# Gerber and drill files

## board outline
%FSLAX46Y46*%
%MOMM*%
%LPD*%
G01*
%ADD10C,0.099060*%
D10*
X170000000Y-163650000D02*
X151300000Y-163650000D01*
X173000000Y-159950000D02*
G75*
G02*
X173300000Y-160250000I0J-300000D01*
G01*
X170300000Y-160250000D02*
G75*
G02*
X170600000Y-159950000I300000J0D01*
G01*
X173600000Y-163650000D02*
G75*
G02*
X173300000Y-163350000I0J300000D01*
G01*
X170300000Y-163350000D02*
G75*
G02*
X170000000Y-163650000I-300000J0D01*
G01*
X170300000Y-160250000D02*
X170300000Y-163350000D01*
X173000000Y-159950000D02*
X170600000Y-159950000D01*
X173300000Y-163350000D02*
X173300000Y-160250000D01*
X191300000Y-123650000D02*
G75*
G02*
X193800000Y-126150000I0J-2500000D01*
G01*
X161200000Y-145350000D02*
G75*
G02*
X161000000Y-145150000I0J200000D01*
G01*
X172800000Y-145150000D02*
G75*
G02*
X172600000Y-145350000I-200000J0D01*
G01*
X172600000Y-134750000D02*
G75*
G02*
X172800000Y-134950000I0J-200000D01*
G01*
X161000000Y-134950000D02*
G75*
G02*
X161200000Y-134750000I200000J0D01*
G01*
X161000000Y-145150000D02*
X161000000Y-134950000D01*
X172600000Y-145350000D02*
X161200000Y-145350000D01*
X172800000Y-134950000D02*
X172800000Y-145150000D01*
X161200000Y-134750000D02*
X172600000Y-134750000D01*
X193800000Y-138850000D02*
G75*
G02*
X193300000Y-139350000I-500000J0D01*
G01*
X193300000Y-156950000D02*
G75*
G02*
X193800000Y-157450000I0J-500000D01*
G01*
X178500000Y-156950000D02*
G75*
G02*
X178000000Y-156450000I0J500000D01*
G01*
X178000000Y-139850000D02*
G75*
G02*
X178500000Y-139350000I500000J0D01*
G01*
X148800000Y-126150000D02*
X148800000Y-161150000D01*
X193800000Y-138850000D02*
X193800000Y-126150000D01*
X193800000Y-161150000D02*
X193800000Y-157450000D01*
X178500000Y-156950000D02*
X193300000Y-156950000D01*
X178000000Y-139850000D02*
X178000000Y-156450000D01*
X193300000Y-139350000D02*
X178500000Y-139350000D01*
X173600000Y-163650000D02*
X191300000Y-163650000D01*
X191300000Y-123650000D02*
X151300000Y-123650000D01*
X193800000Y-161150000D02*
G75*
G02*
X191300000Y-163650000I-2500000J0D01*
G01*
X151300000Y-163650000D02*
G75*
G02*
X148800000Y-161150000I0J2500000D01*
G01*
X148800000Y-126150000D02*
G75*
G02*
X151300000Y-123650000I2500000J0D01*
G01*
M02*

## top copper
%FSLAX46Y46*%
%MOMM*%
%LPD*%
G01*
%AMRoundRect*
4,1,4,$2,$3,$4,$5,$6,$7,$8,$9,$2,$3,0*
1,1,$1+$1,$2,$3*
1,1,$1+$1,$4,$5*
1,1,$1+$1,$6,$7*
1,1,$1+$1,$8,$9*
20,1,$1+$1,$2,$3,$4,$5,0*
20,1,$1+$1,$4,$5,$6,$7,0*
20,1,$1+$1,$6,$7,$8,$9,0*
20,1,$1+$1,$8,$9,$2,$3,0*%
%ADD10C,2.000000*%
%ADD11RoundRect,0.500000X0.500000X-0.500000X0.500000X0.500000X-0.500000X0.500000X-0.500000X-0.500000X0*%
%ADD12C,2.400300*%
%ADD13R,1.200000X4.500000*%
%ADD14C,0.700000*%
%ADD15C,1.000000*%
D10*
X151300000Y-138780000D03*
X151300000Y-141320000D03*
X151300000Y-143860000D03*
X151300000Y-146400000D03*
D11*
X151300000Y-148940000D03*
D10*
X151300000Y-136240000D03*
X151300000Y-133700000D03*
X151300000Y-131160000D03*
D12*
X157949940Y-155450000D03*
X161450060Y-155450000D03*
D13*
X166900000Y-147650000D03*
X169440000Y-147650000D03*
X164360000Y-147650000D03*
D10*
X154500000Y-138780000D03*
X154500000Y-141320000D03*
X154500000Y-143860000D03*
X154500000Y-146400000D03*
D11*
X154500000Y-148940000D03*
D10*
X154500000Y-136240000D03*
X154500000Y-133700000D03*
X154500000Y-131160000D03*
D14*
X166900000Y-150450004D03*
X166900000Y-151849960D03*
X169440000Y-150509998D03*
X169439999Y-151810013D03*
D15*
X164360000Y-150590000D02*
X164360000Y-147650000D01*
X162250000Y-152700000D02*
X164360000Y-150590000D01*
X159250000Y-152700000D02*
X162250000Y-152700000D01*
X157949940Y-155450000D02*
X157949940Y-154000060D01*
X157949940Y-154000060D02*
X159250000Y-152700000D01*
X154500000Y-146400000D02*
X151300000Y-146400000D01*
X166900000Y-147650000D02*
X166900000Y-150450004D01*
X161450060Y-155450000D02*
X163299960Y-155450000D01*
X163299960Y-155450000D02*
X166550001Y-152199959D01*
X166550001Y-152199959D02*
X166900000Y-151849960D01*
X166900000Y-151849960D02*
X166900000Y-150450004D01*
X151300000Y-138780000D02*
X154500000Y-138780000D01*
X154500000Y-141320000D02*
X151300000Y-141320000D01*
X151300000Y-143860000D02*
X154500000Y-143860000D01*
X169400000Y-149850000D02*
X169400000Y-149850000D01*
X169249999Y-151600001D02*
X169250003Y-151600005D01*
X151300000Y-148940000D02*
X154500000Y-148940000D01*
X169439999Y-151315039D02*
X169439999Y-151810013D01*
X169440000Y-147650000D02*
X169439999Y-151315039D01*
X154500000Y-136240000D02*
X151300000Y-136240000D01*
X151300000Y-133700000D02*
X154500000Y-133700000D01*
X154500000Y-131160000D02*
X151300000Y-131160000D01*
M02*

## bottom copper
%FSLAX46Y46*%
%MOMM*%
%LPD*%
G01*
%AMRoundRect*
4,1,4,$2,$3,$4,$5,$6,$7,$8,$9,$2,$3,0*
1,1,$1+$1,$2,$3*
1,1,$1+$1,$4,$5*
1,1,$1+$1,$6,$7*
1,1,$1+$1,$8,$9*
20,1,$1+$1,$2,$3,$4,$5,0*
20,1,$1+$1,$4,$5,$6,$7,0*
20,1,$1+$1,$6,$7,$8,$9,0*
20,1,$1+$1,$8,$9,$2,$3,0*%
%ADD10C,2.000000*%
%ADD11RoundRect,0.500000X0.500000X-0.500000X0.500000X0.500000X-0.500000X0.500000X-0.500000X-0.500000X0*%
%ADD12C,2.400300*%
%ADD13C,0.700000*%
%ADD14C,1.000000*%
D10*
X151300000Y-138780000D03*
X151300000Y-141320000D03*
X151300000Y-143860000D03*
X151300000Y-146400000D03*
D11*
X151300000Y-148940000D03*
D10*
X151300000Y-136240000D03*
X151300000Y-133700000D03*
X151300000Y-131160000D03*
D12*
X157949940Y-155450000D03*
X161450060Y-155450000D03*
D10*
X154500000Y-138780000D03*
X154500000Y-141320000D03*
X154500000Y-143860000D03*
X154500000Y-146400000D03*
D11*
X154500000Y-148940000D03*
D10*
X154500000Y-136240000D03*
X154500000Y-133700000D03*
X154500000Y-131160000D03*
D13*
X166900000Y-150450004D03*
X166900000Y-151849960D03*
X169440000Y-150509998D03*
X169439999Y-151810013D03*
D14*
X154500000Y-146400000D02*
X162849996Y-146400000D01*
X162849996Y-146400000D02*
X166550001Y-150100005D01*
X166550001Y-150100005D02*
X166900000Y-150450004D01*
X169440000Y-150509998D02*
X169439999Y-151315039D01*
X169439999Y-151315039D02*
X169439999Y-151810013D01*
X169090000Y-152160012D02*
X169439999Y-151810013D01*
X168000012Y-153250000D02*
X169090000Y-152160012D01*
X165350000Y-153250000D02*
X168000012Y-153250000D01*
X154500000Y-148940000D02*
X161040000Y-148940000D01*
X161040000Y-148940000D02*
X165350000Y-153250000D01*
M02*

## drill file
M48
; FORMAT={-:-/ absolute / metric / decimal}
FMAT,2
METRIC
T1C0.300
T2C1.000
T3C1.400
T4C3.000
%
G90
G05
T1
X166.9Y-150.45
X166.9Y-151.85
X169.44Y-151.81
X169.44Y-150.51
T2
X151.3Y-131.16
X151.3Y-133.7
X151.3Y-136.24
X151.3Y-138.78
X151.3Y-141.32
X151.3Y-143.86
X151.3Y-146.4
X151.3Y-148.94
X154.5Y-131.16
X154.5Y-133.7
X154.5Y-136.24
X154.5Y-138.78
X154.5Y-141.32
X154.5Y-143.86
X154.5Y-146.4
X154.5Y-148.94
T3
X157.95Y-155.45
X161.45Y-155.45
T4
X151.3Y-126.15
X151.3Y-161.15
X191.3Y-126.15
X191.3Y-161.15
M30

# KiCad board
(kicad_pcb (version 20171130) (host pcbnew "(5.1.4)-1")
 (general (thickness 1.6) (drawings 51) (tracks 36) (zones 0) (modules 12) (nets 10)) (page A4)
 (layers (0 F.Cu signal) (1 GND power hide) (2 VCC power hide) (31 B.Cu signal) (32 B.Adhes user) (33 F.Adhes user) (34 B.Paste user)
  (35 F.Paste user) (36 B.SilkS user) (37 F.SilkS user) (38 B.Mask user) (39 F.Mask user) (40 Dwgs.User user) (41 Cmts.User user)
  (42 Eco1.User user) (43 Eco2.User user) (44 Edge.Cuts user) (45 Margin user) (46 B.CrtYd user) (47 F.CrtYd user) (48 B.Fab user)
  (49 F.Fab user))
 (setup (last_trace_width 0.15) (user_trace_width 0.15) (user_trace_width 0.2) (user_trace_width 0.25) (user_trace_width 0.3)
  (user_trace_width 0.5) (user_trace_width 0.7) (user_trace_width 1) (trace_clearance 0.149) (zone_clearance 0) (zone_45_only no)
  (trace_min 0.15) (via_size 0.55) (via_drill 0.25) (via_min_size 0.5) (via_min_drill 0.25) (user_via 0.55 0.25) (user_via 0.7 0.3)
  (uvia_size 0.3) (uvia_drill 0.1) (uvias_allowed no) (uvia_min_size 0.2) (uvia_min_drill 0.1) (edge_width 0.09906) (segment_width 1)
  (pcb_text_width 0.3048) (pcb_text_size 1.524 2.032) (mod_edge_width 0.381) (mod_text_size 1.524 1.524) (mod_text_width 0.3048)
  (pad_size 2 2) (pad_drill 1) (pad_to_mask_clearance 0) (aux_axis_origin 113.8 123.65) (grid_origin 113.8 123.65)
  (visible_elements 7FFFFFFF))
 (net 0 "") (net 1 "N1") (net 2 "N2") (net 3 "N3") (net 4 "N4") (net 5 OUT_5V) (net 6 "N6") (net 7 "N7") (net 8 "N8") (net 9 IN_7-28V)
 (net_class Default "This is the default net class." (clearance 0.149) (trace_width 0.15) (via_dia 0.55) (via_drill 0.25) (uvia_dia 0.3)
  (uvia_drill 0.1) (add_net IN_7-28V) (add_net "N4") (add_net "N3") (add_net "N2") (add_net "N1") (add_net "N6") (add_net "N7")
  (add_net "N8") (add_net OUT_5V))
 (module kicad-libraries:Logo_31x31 (layer B.Cu) (at 178.8 127.95 180)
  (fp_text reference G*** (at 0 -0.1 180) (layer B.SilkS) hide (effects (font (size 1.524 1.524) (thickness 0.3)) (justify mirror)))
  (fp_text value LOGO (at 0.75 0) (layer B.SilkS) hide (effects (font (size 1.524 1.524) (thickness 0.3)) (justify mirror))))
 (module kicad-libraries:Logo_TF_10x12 (layer F.Cu) (at 181.3 131.65)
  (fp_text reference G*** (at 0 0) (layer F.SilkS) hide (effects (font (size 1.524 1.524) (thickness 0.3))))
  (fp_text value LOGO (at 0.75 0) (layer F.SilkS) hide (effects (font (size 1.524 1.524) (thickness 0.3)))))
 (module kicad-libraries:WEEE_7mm (layer B.Cu) (at 170.7 129.05 180)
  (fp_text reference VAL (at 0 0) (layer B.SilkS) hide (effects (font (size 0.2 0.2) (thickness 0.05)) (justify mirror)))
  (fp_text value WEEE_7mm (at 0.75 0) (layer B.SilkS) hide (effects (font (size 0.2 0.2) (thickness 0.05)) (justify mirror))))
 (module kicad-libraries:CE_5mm (layer B.Cu) (at 164 128.75 180)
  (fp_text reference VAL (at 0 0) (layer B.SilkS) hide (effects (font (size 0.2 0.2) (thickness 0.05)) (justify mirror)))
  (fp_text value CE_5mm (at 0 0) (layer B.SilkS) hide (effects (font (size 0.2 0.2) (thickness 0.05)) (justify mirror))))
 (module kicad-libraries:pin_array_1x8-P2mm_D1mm (layer F.Cu) (at 151.3 140.05 90)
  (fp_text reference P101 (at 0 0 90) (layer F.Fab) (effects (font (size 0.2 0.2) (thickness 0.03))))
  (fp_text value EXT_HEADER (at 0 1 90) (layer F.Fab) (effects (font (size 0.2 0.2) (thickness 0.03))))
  (pad 5 thru_hole circle (at 1.27 0 90) (size 2 2) (drill 1) (layers *.Cu *.Mask) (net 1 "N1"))
  (pad 4 thru_hole circle (at -1.27 0 90) (size 2 2) (drill 1) (layers *.Cu *.Mask) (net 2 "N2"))
  (pad 3 thru_hole circle (at -3.81 0 90) (size 2 2) (drill 1) (layers *.Cu *.Mask) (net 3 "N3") (zone_connect 1) (thermal_width 0.7)
   (thermal_gap 0.2))
  (pad 2 thru_hole circle (at -6.35 0 90) (size 2 2) (drill 1) (layers *.Cu *.Mask) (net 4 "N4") (zone_connect 1) (thermal_width 0.7)
   (thermal_gap 0.2))
  (pad 1 thru_hole roundrect (at -8.89 0 90) (size 2 2) (drill 1) (layers *.Cu *.Mask) (roundrect_rratio 0.25) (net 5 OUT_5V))
  (pad 6 thru_hole circle (at 3.81 0 90) (size 2 2) (drill 1) (layers *.Cu *.Mask) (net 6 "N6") (zone_connect 1) (thermal_width 0.7)
   (thermal_gap 0.2))
  (pad 7 thru_hole circle (at 6.35 0 90) (size 2 2) (drill 1) (layers *.Cu *.Mask) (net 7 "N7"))
  (pad 8 thru_hole circle (at 8.89 0 90) (size 2 2) (drill 1) (layers *.Cu *.Mask) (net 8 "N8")))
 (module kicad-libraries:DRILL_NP (layer F.Cu) (at 151.3 126.15)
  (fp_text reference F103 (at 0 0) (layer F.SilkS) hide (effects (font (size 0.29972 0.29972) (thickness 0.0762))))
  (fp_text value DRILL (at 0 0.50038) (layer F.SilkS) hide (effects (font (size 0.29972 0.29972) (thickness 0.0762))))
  (pad "" np_thru_hole circle (at 0 0) (size 2.99974 2.99974) (drill 2.99974) (layers *.Cu *.Mask F.SilkS) (clearance 0.89916)))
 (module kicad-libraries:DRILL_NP (layer F.Cu) (at 151.3 161.15)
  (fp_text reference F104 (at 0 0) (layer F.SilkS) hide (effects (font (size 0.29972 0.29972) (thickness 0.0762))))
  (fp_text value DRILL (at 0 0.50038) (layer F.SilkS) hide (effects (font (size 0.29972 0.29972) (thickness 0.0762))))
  (pad "" np_thru_hole circle (at 0 0) (size 2.99974 2.99974) (drill 2.99974) (layers *.Cu *.Mask F.SilkS) (clearance 0.89916)))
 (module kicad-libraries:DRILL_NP (layer F.Cu) (at 191.3 161.15)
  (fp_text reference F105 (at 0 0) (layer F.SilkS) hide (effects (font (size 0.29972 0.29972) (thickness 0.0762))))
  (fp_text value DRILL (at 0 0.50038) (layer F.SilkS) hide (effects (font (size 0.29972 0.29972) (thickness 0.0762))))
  (pad "" np_thru_hole circle (at 0 0) (size 2.99974 2.99974) (drill 2.99974) (layers *.Cu *.Mask F.SilkS) (clearance 0.89916)))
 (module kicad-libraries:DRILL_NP (layer F.Cu) (at 191.3 126.15)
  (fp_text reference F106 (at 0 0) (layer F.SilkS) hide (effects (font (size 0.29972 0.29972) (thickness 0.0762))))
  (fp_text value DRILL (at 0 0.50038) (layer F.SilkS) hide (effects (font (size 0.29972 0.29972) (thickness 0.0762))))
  (pad "" np_thru_hole circle (at 0 0) (size 2.99974 2.99974) (drill 2.99974) (layers *.Cu *.Mask F.SilkS) (clearance 0.89916)))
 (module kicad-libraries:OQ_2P (layer F.Cu) (at 159.7 155.45)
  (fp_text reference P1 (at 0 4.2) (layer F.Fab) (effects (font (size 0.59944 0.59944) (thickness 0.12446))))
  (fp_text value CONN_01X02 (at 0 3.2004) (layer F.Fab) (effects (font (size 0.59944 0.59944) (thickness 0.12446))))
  (pad 1 thru_hole circle (at -1.75006 0) (size 2.4003 2.4003) (drill 1.39954) (layers *.Cu *.Mask F.SilkS) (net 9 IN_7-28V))
  (pad 2 thru_hole circle (at 1.75006 0) (size 2.4003 2.4003) (drill 1.39954) (layers *.Cu *.Mask F.SilkS) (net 4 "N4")))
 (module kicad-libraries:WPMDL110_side (layer F.Cu) (at 166.9 143.85 90)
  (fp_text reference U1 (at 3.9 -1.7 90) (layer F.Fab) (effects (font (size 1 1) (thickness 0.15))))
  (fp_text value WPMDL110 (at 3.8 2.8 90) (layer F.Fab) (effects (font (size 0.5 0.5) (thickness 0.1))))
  (pad 2 smd rect (at -3.8 0 90) (size 4.5 1.2) (layers F.Cu F.Paste F.Mask) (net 4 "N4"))
  (pad 3 smd rect (at -3.8 2.54 90) (size 4.5 1.2) (layers F.Cu F.Paste F.Mask) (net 5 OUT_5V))
  (pad 1 smd rect (at -3.8 -2.54 90) (size 4.5 1.2) (layers F.Cu F.Paste F.Mask) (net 9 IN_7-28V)))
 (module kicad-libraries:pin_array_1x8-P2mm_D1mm (layer F.Cu) (at 154.5 140.05 90)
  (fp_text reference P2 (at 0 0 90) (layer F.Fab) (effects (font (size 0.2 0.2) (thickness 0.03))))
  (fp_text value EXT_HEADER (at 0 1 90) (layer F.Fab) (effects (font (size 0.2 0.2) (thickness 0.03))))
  (pad 5 thru_hole circle (at 1.27 0 90) (size 2 2) (drill 1) (layers *.Cu *.Mask) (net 1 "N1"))
  (pad 4 thru_hole circle (at -1.27 0 90) (size 2 2) (drill 1) (layers *.Cu *.Mask) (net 2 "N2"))
  (pad 3 thru_hole circle (at -3.81 0 90) (size 2 2) (drill 1) (layers *.Cu *.Mask) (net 3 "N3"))
  (pad 2 thru_hole circle (at -6.35 0 90) (size 2 2) (drill 1) (layers *.Cu *.Mask) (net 4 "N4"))
  (pad 1 thru_hole roundrect (at -8.89 0 90) (size 2 2) (drill 1) (layers *.Cu *.Mask) (roundrect_rratio 0.25) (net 5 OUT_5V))
  (pad 6 thru_hole circle (at 3.81 0 90) (size 2 2) (drill 1) (layers *.Cu *.Mask) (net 6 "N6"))
  (pad 7 thru_hole circle (at 6.35 0 90) (size 2 2) (drill 1) (layers *.Cu *.Mask) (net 7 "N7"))
  (pad 8 thru_hole circle (at 8.89 0 90) (size 2 2) (drill 1) (layers *.Cu *.Mask) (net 8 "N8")))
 (gr_line (start 170 163.65) (end 151.3 163.65) (layer Edge.Cuts) (width 0.09906))
 (gr_arc (start 173 160.25) (end 173.3 160.25) (angle -90) (layer Edge.Cuts) (width 0.09906))
 (gr_arc (start 170.6 160.25) (end 170.6 159.95) (angle -90) (layer Edge.Cuts) (width 0.09906))
 (gr_arc (start 173.6 163.35) (end 173.3 163.35) (angle -90) (layer Edge.Cuts) (width 0.09906))
 (gr_arc (start 170 163.35) (end 170 163.65) (angle -90) (layer Edge.Cuts) (width 0.09906))
 (gr_line (start 170.3 160.25) (end 170.3 163.35) (layer Edge.Cuts) (width 0.09906))
 (gr_line (start 173 159.95) (end 170.6 159.95) (layer Edge.Cuts) (width 0.09906))
 (gr_line (start 173.3 163.35) (end 173.3 160.25) (layer Edge.Cuts) (width 0.09906))
 (gr_arc (start 191.3 126.15) (end 193.8 126.15) (angle -90) (layer Edge.Cuts) (width 0.09906))
 (gr_arc (start 161.2 145.15) (end 161 145.15) (angle -90) (layer Edge.Cuts) (width 0.09906))
 (gr_arc (start 172.6 145.15) (end 172.6 145.35) (angle -90) (layer Edge.Cuts) (width 0.09906))
 (gr_arc (start 172.6 134.95) (end 172.8 134.95) (angle -90) (layer Edge.Cuts) (width 0.09906))
 (gr_arc (start 161.2 134.95) (end 161.2 134.75) (angle -90) (layer Edge.Cuts) (width 0.09906))
 (gr_line (start 161 145.15) (end 161 134.95) (layer Edge.Cuts) (width 0.09906))
 (gr_line (start 172.6 145.35) (end 161.2 145.35) (layer Edge.Cuts) (width 0.09906))
 (gr_line (start 172.8 134.95) (end 172.8 145.15) (layer Edge.Cuts) (width 0.09906))
 (gr_line (start 161.2 134.75) (end 172.6 134.75) (layer Edge.Cuts) (width 0.09906))
 (gr_arc (start 193.3 138.85) (end 193.3 139.35) (angle -90) (layer Edge.Cuts) (width 0.09906))
 (gr_arc (start 193.3 157.45) (end 193.8 157.45) (angle -90) (layer Edge.Cuts) (width 0.09906))
 (gr_arc (start 178.5 156.45) (end 178 156.45) (angle -90) (layer Edge.Cuts) (width 0.09906))
 (gr_arc (start 178.5 139.85) (end 178.5 139.35) (angle -90) (layer Edge.Cuts) (width 0.09906))
 (gr_line (start 148.8 126.15) (end 148.8 161.15) (layer Edge.Cuts) (width 0.09906))
 (gr_line (start 193.8 138.85) (end 193.8 126.15) (layer Edge.Cuts) (width 0.09906))
 (gr_line (start 193.8 161.15) (end 193.8 157.45) (layer Edge.Cuts) (width 0.09906))
 (gr_line (start 178.5 156.95) (end 193.3 156.95) (layer Edge.Cuts) (width 0.09906))
 (gr_line (start 178 139.85) (end 178 156.45) (layer Edge.Cuts) (width 0.09906))
 (gr_line (start 193.3 139.35) (end 178.5 139.35) (layer Edge.Cuts) (width 0.09906))
 (gr_line (start 173.6 163.65) (end 191.3 163.65) (layer Edge.Cuts) (width 0.09906))
 (gr_line (start 191.3 123.65) (end 151.3 123.65) (layer Edge.Cuts) (width 0.09906))
 (gr_arc (start 191.3 161.15) (end 191.3 163.65) (angle -90) (layer Edge.Cuts) (width 0.09906))
 (gr_arc (start 151.3 161.15) (end 148.8 161.15) (angle -90) (layer Edge.Cuts) (width 0.09906))
 (gr_arc (start 151.3 126.15) (end 151.3 123.65) (angle -90) (layer Edge.Cuts) (width 0.09906))
 (segment (start 164.36 150.59) (end 164.36 147.65) (width 1) (layer F.Cu) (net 9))
 (segment (start 162.25 152.7) (end 164.36 150.59) (width 1) (layer F.Cu) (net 9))
 (segment (start 159.25 152.7) (end 162.25 152.7) (width 1) (layer F.Cu) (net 9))
 (segment (start 157.94994 155.45) (end 157.94994 154.00006) (width 1) (layer F.Cu) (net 9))
 (segment (start 157.94994 154.00006) (end 159.25 152.7) (width 1) (layer F.Cu) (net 9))
 (segment (start 154.5 146.4) (end 151.3 146.4) (width 1) (layer F.Cu) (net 4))
 (via (at 166.9 150.450004) (size 0.7) (drill 0.3) (layers F.Cu B.Cu) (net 4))
 (segment (start 166.9 147.65) (end 166.9 150.450004) (width 1) (layer F.Cu) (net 4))
 (segment (start 154.5 146.4) (end 162.849996 146.4) (width 1) (layer B.Cu) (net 4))
 (segment (start 162.849996 146.4) (end 166.550001 150.100005) (width 1) (layer B.Cu) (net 4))
 (segment (start 166.550001 150.100005) (end 166.9 150.450004) (width 1) (layer B.Cu) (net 4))
 (via (at 166.9 151.84996) (size 0.7) (drill 0.3) (layers F.Cu B.Cu) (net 4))
 (segment (start 161.45006 155.45) (end 163.29996 155.45) (width 1) (layer F.Cu) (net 4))
 (segment (start 163.29996 155.45) (end 166.550001 152.199959) (width 1) (layer F.Cu) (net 4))
 (segment (start 166.550001 152.199959) (end 166.9 151.84996) (width 1) (layer F.Cu) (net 4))
 (segment (start 166.9 151.84996) (end 166.9 150.450004) (width 1) (layer F.Cu) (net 4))
 (segment (start 151.3 138.78) (end 154.5 138.78) (width 1) (layer F.Cu) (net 1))
 (segment (start 154.5 141.32) (end 151.3 141.32) (width 1) (layer F.Cu) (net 2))
 (segment (start 151.3 143.86) (end 154.5 143.86) (width 1) (layer F.Cu) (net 3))
 (segment (start 169.4 149.85) (end 169.4 149.85) (width 1) (layer F.Cu) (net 5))
 (segment (start 169.249999 151.600001) (end 169.250003 151.600005) (width 1) (layer F.Cu) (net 5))
 (segment (start 151.3 148.94) (end 154.5 148.94) (width 1) (layer F.Cu) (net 5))
 (via (at 169.44 150.509998) (size 0.7) (drill 0.3) (layers F.Cu B.Cu) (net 5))
 (via (at 169.439999 151.810013) (size 0.7) (drill 0.3) (layers F.Cu B.Cu) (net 5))
 (segment (start 169.439999 151.315039) (end 169.439999 151.810013) (width 1) (layer F.Cu) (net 5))
 (segment (start 169.44 150.509998) (end 169.439999 151.315039) (width 1) (layer B.Cu) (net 5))
 (segment (start 169.439999 151.315039) (end 169.439999 151.810013) (width 1) (layer B.Cu) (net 5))
 (segment (start 169.44 147.65) (end 169.439999 151.315039) (width 1) (layer F.Cu) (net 5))
 (segment (start 169.09 152.160012) (end 169.439999 151.810013) (width 1) (layer B.Cu) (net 5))
 (segment (start 168.000012 153.25) (end 169.09 152.160012) (width 1) (layer B.Cu) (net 5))
 (segment (start 165.35 153.25) (end 168.000012 153.25) (width 1) (layer B.Cu) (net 5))
 (segment (start 154.5 148.94) (end 161.04 148.94) (width 1) (layer B.Cu) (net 5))
 (segment (start 161.04 148.94) (end 165.35 153.25) (width 1) (layer B.Cu) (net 5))
 (segment (start 154.5 136.24) (end 151.3 136.24) (width 1) (layer F.Cu) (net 6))
 (segment (start 151.3 133.7) (end 154.5 133.7) (width 1) (layer F.Cu) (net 7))
 (segment (start 154.5 131.16) (end 151.3 131.16) (width 1) (layer F.Cu) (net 8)))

